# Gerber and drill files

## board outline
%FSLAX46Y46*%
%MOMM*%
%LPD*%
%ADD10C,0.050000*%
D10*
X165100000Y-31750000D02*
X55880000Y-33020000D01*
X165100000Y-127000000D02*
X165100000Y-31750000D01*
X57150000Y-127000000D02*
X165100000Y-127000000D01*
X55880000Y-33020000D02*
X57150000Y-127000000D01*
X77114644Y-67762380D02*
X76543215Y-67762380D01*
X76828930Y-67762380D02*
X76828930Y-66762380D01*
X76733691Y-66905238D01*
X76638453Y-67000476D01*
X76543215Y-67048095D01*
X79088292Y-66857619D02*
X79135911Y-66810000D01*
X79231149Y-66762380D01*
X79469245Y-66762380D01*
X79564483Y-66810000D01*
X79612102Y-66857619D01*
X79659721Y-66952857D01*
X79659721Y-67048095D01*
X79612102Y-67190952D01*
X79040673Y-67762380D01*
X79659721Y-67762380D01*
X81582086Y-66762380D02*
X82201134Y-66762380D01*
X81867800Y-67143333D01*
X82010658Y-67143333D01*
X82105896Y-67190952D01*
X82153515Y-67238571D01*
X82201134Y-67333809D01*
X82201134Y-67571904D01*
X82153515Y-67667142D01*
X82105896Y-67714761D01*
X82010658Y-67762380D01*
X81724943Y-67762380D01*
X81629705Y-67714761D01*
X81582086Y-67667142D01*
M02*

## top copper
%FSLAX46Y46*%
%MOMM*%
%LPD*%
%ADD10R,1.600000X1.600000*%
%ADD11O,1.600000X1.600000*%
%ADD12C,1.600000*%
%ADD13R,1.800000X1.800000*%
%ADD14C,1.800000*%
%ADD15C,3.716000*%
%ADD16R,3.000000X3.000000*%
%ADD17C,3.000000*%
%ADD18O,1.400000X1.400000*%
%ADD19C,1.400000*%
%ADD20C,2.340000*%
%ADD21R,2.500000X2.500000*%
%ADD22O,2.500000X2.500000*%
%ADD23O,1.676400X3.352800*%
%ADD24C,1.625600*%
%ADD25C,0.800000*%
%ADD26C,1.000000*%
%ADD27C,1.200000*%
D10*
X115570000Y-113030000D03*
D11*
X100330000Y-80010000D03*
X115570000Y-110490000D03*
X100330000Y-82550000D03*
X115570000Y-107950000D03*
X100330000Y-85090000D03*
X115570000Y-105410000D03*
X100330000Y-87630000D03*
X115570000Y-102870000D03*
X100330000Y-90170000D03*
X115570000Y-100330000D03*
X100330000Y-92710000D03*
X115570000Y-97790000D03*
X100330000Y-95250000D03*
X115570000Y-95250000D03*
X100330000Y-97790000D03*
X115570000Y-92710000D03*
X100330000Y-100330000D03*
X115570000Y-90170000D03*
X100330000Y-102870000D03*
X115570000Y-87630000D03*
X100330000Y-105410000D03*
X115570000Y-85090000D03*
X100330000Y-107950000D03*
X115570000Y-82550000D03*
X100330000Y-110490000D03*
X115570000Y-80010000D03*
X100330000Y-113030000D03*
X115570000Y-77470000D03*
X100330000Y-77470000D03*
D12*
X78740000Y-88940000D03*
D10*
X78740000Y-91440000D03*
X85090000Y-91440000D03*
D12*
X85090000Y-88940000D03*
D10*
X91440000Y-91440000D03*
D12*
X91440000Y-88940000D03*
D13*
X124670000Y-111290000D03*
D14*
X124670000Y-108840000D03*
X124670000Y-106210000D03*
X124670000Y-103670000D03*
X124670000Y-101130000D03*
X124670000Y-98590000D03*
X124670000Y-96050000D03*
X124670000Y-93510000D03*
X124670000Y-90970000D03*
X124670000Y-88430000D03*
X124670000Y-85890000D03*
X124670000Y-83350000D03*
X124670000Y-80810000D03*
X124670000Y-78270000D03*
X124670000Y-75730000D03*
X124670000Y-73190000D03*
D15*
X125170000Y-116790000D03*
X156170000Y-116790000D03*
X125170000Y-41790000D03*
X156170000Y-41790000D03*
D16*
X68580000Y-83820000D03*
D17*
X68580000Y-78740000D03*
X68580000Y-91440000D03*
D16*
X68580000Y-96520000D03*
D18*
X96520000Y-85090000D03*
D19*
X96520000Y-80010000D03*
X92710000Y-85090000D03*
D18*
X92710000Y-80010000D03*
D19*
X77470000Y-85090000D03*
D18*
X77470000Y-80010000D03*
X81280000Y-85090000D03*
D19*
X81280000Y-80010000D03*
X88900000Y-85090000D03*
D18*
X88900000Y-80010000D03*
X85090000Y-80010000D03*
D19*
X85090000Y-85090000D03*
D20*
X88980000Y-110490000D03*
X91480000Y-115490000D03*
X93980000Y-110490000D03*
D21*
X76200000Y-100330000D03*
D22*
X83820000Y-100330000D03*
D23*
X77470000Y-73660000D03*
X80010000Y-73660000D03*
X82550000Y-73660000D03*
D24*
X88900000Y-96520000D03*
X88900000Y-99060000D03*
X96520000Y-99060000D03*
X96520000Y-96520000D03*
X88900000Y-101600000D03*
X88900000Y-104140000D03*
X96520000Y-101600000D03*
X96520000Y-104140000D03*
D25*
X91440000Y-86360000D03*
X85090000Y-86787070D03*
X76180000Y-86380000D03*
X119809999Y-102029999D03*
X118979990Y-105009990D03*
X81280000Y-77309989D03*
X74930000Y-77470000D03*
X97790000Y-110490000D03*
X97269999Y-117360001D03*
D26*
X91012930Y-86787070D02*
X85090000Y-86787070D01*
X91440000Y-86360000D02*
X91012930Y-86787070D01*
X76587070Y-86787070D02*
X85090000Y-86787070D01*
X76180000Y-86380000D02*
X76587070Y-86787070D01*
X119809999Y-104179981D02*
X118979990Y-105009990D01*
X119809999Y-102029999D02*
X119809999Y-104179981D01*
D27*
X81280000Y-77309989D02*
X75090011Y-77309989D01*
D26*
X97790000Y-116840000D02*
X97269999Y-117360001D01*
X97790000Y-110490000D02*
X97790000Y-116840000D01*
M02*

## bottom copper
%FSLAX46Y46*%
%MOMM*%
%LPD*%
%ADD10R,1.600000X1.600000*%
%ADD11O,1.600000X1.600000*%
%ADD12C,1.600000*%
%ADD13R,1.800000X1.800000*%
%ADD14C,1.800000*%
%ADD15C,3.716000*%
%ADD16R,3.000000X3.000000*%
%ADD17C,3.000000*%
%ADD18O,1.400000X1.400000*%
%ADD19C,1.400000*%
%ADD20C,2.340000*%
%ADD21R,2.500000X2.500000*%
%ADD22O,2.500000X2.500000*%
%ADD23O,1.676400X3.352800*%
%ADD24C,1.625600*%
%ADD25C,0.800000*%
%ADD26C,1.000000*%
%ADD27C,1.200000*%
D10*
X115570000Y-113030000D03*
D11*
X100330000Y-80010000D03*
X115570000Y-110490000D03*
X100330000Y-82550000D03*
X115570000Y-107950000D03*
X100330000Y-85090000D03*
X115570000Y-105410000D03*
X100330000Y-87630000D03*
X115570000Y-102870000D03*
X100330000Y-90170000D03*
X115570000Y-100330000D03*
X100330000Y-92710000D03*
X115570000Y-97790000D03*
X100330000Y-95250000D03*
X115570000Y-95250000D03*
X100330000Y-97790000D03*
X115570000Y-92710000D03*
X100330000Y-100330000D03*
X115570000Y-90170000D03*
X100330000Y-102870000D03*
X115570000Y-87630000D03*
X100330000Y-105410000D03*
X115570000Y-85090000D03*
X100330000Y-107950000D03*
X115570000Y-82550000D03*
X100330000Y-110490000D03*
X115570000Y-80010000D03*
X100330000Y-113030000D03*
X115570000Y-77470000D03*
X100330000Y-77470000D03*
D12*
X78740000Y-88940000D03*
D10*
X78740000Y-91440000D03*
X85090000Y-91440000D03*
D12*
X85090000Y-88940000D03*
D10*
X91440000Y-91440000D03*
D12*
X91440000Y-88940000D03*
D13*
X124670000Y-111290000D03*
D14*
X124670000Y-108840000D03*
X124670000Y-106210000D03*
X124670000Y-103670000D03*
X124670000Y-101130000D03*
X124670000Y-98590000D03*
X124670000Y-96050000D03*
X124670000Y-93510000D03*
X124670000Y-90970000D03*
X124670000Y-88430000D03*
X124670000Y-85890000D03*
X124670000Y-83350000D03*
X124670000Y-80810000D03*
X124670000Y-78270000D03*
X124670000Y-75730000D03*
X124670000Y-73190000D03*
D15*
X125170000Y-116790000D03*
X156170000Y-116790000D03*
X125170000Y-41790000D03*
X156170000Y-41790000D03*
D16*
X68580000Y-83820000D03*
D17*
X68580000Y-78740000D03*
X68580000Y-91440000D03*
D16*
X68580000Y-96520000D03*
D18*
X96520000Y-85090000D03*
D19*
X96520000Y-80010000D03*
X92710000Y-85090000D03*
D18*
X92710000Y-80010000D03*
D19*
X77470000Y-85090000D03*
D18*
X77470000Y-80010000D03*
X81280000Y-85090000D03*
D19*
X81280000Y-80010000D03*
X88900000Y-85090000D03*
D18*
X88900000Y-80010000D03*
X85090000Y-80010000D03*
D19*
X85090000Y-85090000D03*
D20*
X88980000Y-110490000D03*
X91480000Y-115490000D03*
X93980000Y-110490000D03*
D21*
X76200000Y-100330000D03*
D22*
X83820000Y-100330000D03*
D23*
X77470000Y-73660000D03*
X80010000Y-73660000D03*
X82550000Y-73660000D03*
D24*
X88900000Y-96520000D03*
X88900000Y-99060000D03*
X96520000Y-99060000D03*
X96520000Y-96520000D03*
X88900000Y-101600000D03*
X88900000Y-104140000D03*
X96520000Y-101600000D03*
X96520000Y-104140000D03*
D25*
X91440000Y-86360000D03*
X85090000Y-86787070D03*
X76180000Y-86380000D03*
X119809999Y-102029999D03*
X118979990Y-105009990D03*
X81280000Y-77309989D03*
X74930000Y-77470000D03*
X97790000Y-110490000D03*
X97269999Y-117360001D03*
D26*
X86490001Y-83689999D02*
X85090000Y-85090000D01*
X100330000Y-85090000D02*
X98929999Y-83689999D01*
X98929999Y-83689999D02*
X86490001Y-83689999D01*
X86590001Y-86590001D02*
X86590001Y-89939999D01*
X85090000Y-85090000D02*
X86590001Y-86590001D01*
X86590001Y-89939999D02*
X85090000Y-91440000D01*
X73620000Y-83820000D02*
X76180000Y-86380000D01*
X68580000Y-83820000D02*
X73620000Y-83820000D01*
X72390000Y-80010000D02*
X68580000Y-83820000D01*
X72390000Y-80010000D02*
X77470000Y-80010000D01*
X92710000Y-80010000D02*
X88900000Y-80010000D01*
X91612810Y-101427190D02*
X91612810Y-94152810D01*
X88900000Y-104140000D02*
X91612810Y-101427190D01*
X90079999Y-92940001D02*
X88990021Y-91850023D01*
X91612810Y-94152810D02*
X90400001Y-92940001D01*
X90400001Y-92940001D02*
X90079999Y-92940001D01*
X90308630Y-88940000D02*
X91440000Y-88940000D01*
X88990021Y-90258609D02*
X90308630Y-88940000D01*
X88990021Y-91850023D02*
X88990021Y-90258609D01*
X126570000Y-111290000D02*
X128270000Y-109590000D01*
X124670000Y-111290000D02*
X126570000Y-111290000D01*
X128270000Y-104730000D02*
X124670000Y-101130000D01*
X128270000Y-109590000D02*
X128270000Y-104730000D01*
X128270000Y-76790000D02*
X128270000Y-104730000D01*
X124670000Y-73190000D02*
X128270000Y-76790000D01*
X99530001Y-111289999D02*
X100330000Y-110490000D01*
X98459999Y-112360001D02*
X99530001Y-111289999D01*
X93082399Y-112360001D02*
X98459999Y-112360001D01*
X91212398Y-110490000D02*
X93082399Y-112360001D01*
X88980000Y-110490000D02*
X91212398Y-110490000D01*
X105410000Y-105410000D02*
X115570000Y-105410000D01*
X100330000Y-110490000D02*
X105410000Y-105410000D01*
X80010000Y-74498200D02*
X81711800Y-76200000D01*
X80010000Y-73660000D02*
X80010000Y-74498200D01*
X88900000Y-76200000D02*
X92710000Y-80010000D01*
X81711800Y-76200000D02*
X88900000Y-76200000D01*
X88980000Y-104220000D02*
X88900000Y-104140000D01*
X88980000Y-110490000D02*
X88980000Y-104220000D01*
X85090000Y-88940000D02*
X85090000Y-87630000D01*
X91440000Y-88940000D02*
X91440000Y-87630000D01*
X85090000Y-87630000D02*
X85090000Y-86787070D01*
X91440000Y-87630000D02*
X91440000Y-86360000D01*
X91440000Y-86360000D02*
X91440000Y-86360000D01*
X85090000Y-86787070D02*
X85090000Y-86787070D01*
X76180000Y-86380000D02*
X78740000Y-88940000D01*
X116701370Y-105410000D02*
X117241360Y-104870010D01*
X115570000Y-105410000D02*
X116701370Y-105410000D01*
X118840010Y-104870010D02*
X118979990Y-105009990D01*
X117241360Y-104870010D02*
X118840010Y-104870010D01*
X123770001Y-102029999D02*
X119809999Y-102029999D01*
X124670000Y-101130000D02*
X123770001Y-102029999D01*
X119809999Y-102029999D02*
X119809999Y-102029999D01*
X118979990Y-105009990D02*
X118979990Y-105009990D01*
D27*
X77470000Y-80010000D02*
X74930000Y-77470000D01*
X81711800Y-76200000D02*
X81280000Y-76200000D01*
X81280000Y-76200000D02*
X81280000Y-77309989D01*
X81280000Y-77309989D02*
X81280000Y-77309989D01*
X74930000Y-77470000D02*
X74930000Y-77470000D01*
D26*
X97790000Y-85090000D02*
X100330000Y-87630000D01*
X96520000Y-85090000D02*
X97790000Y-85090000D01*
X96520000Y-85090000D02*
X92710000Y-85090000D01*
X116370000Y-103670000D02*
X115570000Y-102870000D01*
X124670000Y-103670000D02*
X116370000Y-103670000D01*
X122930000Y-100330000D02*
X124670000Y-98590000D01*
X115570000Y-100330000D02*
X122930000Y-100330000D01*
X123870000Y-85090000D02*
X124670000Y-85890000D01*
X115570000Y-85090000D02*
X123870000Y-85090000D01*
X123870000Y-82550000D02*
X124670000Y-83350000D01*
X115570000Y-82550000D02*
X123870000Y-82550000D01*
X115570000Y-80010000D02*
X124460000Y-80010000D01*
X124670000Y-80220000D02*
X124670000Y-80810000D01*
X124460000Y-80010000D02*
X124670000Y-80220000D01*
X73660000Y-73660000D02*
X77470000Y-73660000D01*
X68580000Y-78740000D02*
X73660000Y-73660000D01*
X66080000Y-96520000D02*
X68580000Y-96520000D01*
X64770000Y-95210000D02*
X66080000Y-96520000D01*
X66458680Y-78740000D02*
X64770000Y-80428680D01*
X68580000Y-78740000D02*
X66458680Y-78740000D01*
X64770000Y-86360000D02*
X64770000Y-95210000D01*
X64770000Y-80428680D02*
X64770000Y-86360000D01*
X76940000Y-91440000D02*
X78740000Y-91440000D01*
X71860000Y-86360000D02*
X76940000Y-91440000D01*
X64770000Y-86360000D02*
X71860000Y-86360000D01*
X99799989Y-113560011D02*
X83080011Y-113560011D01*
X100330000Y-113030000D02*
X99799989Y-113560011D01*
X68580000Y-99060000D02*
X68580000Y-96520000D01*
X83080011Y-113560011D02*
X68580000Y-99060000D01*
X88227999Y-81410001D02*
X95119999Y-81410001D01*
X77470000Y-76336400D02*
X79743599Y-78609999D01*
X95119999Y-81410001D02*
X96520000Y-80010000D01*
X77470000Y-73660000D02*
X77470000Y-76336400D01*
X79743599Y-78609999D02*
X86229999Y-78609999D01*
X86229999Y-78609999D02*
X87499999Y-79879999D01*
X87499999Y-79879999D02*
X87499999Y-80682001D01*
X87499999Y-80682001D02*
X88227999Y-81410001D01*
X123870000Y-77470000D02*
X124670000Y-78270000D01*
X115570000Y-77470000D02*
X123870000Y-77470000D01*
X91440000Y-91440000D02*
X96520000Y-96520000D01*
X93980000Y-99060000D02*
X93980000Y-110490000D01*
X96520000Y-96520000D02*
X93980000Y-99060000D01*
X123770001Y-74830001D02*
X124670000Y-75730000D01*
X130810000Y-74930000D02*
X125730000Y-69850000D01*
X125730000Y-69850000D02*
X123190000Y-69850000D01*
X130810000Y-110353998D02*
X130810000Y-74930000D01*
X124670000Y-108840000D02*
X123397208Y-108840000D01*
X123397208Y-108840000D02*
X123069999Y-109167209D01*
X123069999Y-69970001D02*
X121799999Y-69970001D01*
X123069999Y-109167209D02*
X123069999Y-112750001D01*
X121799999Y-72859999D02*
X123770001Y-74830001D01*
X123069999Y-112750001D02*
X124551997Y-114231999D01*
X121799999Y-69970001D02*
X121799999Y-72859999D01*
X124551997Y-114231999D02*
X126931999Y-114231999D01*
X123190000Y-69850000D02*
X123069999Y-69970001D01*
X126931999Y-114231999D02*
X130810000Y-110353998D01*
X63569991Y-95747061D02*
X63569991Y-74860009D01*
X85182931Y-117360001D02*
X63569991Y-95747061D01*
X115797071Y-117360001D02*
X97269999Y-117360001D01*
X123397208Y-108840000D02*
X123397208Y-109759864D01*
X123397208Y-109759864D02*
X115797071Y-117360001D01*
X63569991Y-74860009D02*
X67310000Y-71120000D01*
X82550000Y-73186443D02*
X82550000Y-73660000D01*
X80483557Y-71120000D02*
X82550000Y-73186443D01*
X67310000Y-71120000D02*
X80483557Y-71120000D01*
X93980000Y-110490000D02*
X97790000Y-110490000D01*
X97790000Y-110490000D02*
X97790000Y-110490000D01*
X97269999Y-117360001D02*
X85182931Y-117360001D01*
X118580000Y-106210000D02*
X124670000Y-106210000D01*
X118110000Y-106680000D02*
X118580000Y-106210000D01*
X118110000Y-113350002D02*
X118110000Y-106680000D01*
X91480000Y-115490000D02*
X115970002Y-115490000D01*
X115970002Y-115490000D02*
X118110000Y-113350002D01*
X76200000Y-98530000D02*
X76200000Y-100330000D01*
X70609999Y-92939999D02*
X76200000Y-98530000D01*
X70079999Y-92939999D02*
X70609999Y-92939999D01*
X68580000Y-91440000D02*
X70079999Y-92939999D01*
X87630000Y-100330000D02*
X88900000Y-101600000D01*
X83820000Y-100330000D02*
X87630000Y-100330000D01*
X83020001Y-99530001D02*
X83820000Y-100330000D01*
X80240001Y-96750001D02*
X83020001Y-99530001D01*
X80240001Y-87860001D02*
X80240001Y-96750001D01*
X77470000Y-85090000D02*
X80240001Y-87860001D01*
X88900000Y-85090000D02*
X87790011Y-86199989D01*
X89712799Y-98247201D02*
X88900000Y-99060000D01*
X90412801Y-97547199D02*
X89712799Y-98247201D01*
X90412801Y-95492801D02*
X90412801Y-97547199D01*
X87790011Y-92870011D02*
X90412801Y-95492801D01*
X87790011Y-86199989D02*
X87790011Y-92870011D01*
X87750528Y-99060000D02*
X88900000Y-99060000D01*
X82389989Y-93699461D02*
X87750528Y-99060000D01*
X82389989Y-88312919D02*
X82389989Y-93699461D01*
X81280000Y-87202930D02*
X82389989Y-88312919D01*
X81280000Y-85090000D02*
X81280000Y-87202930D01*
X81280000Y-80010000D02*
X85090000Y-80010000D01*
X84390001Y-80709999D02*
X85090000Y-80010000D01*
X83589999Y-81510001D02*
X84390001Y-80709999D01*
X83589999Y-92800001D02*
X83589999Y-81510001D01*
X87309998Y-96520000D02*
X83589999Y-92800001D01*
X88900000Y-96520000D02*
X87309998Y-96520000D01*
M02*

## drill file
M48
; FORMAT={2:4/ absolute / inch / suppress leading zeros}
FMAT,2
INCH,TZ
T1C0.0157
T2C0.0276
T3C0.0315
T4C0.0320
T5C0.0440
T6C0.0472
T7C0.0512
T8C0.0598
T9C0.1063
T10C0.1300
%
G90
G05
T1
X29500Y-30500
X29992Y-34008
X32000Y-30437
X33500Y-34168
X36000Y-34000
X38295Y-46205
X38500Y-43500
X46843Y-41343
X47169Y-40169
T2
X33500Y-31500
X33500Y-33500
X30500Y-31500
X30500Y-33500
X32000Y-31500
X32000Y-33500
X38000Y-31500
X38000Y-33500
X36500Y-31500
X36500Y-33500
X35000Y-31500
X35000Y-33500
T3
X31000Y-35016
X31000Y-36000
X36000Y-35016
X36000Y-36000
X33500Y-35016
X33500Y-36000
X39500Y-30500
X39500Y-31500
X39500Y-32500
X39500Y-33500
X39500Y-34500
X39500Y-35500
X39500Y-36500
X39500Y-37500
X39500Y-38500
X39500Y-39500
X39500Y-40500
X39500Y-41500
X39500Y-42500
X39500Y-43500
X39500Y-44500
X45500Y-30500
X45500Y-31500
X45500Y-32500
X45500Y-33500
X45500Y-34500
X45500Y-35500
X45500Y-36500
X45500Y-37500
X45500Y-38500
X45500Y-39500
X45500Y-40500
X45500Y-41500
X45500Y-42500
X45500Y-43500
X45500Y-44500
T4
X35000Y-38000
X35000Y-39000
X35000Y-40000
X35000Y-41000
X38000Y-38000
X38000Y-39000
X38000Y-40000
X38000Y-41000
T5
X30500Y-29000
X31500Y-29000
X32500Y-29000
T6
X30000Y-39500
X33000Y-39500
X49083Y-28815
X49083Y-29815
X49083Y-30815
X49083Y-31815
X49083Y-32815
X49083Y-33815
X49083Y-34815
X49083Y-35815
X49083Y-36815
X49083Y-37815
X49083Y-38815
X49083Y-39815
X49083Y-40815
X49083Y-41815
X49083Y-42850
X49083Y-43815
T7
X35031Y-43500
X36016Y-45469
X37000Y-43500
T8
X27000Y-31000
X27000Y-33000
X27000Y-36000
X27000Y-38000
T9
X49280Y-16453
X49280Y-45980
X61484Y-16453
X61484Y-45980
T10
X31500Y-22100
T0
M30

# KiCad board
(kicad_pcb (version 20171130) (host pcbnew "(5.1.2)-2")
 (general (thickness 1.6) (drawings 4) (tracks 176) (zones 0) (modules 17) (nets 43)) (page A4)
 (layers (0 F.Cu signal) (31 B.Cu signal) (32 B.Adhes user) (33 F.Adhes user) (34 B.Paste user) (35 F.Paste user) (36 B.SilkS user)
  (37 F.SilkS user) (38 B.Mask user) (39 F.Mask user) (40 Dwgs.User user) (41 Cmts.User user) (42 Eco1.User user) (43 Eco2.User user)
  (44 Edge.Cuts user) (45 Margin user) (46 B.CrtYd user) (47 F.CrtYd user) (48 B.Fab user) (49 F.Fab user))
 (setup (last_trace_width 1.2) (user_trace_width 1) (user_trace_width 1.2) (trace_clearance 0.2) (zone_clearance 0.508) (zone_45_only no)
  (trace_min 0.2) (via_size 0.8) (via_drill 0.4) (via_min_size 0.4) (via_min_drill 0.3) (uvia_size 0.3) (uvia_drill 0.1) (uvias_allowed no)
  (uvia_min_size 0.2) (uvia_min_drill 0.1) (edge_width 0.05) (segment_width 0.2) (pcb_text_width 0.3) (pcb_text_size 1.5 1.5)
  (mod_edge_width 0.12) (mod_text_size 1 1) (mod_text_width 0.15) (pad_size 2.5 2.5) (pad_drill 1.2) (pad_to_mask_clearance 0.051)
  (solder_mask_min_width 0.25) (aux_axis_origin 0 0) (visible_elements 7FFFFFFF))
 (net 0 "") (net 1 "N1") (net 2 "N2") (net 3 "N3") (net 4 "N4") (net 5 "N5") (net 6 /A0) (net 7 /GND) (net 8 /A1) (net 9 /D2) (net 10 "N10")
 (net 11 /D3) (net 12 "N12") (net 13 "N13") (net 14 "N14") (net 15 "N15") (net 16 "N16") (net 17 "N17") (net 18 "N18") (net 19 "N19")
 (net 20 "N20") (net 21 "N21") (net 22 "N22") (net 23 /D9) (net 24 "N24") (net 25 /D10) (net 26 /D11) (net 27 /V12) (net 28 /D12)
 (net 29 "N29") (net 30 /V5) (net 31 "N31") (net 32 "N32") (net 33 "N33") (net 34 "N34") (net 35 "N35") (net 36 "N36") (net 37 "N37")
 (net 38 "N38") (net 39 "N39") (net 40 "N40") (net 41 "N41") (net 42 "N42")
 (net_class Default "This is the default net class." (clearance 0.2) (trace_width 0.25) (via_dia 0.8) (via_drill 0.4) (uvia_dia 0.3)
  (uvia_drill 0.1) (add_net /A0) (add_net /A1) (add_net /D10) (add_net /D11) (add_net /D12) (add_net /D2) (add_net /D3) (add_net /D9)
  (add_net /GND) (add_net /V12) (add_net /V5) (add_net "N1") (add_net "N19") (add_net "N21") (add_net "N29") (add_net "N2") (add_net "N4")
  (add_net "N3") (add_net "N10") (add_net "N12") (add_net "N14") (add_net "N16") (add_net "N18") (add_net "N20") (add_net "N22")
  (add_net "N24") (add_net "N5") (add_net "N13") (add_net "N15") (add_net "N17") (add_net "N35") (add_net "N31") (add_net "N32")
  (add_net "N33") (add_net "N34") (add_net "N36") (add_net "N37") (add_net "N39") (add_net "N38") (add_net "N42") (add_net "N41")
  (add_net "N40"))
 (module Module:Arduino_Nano (layer F.Cu) (at 115.57 113.03 180)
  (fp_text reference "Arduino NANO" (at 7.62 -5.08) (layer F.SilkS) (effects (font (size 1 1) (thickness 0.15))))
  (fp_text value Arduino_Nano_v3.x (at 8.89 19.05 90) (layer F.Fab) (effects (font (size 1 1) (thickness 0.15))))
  (pad 1 thru_hole rect (at 0 0 180) (size 1.6 1.6) (drill 0.8) (layers *.Cu *.Mask) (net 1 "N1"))
  (pad 17 thru_hole oval (at 15.24 33.02 180) (size 1.6 1.6) (drill 0.8) (layers *.Cu *.Mask) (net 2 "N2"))
  (pad 2 thru_hole oval (at 0 2.54 180) (size 1.6 1.6) (drill 0.8) (layers *.Cu *.Mask) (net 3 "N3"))
  (pad 18 thru_hole oval (at 15.24 30.48 180) (size 1.6 1.6) (drill 0.8) (layers *.Cu *.Mask) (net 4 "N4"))
  (pad 3 thru_hole oval (at 0 5.08 180) (size 1.6 1.6) (drill 0.8) (layers *.Cu *.Mask) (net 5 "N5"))
  (pad 19 thru_hole oval (at 15.24 27.94 180) (size 1.6 1.6) (drill 0.8) (layers *.Cu *.Mask) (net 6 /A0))
  (pad 4 thru_hole oval (at 0 7.62 180) (size 1.6 1.6) (drill 0.8) (layers *.Cu *.Mask) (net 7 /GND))
  (pad 20 thru_hole oval (at 15.24 25.4 180) (size 1.6 1.6) (drill 0.8) (layers *.Cu *.Mask) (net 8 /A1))
  (pad 5 thru_hole oval (at 0 10.16 180) (size 1.6 1.6) (drill 0.8) (layers *.Cu *.Mask) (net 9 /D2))
  (pad 21 thru_hole oval (at 15.24 22.86 180) (size 1.6 1.6) (drill 0.8) (layers *.Cu *.Mask) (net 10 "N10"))
  (pad 6 thru_hole oval (at 0 12.7 180) (size 1.6 1.6) (drill 0.8) (layers *.Cu *.Mask) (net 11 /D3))
  (pad 22 thru_hole oval (at 15.24 20.32 180) (size 1.6 1.6) (drill 0.8) (layers *.Cu *.Mask) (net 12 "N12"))
  (pad 7 thru_hole oval (at 0 15.24 180) (size 1.6 1.6) (drill 0.8) (layers *.Cu *.Mask) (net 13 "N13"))
  (pad 23 thru_hole oval (at 15.24 17.78 180) (size 1.6 1.6) (drill 0.8) (layers *.Cu *.Mask) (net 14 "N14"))
  (pad 8 thru_hole oval (at 0 17.78 180) (size 1.6 1.6) (drill 0.8) (layers *.Cu *.Mask) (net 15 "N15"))
  (pad 24 thru_hole oval (at 15.24 15.24 180) (size 1.6 1.6) (drill 0.8) (layers *.Cu *.Mask) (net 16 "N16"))
  (pad 9 thru_hole oval (at 0 20.32 180) (size 1.6 1.6) (drill 0.8) (layers *.Cu *.Mask) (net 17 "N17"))
  (pad 25 thru_hole oval (at 15.24 12.7 180) (size 1.6 1.6) (drill 0.8) (layers *.Cu *.Mask) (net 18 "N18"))
  (pad 10 thru_hole oval (at 0 22.86 180) (size 1.6 1.6) (drill 0.8) (layers *.Cu *.Mask) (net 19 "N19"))
  (pad 26 thru_hole oval (at 15.24 10.16 180) (size 1.6 1.6) (drill 0.8) (layers *.Cu *.Mask) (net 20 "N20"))
  (pad 11 thru_hole oval (at 0 25.4 180) (size 1.6 1.6) (drill 0.8) (layers *.Cu *.Mask) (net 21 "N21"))
  (pad 27 thru_hole oval (at 15.24 7.62 180) (size 1.6 1.6) (drill 0.8) (layers *.Cu *.Mask) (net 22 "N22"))
  (pad 12 thru_hole oval (at 0 27.94 180) (size 1.6 1.6) (drill 0.8) (layers *.Cu *.Mask) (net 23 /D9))
  (pad 28 thru_hole oval (at 15.24 5.08 180) (size 1.6 1.6) (drill 0.8) (layers *.Cu *.Mask) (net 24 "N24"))
  (pad 13 thru_hole oval (at 0 30.48 180) (size 1.6 1.6) (drill 0.8) (layers *.Cu *.Mask) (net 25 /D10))
  (pad 29 thru_hole oval (at 15.24 2.54 180) (size 1.6 1.6) (drill 0.8) (layers *.Cu *.Mask) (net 7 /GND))
  (pad 14 thru_hole oval (at 0 33.02 180) (size 1.6 1.6) (drill 0.8) (layers *.Cu *.Mask) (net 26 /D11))
  (pad 30 thru_hole oval (at 15.24 0 180) (size 1.6 1.6) (drill 0.8) (layers *.Cu *.Mask) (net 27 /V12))
  (pad 15 thru_hole oval (at 0 35.56 180) (size 1.6 1.6) (drill 0.8) (layers *.Cu *.Mask) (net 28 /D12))
  (pad 16 thru_hole oval (at 15.24 35.56 180) (size 1.6 1.6) (drill 0.8) (layers *.Cu *.Mask) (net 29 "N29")))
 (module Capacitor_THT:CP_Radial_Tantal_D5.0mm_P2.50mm (layer F.Cu) (at 78.74 91.44 90)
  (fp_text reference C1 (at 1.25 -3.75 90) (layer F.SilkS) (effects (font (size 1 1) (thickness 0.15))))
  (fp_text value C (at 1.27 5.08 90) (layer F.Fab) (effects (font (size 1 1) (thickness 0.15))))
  (pad 2 thru_hole circle (at 2.5 0 90) (size 1.6 1.6) (drill 0.8) (layers *.Cu *.Mask) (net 7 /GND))
  (pad 1 thru_hole rect (at 0 0 90) (size 1.6 1.6) (drill 0.8) (layers *.Cu *.Mask) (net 27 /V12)))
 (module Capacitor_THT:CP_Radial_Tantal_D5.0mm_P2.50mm (layer F.Cu) (at 85.09 91.44 90)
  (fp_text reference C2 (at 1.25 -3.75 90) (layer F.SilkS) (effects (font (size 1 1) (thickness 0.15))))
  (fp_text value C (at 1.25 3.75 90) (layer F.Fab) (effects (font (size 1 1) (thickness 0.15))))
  (pad 1 thru_hole rect (at 0 0 90) (size 1.6 1.6) (drill 0.8) (layers *.Cu *.Mask) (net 6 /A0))
  (pad 2 thru_hole circle (at 2.5 0 90) (size 1.6 1.6) (drill 0.8) (layers *.Cu *.Mask) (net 7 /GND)))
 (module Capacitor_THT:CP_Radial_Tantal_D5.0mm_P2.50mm (layer F.Cu) (at 91.44 91.44 90)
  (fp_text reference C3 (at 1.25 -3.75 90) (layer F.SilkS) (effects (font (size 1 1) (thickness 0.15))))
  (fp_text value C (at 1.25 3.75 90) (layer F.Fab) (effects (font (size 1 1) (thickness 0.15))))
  (pad 1 thru_hole rect (at 0 0 90) (size 1.6 1.6) (drill 0.8) (layers *.Cu *.Mask) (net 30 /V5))
  (pad 2 thru_hole circle (at 2.5 0 90) (size 1.6 1.6) (drill 0.8) (layers *.Cu *.Mask) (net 7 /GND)))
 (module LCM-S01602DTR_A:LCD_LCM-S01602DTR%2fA (layer F.Cu) (at 140.97 78.74 90)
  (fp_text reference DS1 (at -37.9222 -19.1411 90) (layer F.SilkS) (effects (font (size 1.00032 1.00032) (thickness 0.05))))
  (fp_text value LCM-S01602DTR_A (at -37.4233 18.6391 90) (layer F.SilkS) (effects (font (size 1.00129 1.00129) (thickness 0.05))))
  (pad 1 thru_hole rect (at -32.55 -16.3 90) (size 1.8 1.8) (drill 1.2) (layers *.Cu *.Mask) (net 7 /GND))
  (pad 2 thru_hole circle (at -30.1 -16.3 90) (size 1.8 1.8) (drill 1.2) (layers *.Cu *.Mask) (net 30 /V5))
  (pad 3 thru_hole circle (at -27.47 -16.3 90) (size 1.8 1.8) (drill 1.2) (layers *.Cu *.Mask) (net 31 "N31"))
  (pad 4 thru_hole circle (at -24.93 -16.3 90) (size 1.8 1.8) (drill 1.2) (layers *.Cu *.Mask) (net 9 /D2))
  (pad 5 thru_hole circle (at -22.39 -16.3 90) (size 1.8 1.8) (drill 1.2) (layers *.Cu *.Mask) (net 7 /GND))
  (pad 6 thru_hole circle (at -19.85 -16.3 90) (size 1.8 1.8) (drill 1.2) (layers *.Cu *.Mask) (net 11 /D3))
  (pad 7 thru_hole circle (at -17.31 -16.3 90) (size 1.8 1.8) (drill 1.2) (layers *.Cu *.Mask) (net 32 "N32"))
  (pad 8 thru_hole circle (at -14.77 -16.3 90) (size 1.8 1.8) (drill 1.2) (layers *.Cu *.Mask) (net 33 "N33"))
  (pad 9 thru_hole circle (at -12.23 -16.3 90) (size 1.8 1.8) (drill 1.2) (layers *.Cu *.Mask) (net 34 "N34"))
  (pad 10 thru_hole circle (at -9.69 -16.3 90) (size 1.8 1.8) (drill 1.2) (layers *.Cu *.Mask) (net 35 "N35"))
  (pad 11 thru_hole circle (at -7.15 -16.3 90) (size 1.8 1.8) (drill 1.2) (layers *.Cu *.Mask) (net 23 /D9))
  (pad 12 thru_hole circle (at -4.61 -16.3 90) (size 1.8 1.8) (drill 1.2) (layers *.Cu *.Mask) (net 25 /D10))
  (pad 13 thru_hole circle (at -2.07 -16.3 90) (size 1.8 1.8) (drill 1.2) (layers *.Cu *.Mask) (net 26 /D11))
  (pad 14 thru_hole circle (at 0.47 -16.3 90) (size 1.8 1.8) (drill 1.2) (layers *.Cu *.Mask) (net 28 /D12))
  (pad 15 thru_hole circle (at 3.01 -16.3 90) (size 1.8 1.8) (drill 1.2) (layers *.Cu *.Mask) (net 30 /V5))
  (pad 16 thru_hole circle (at 5.55 -16.3 90) (size 1.8 1.8) (drill 1.2) (layers *.Cu *.Mask) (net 7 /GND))
  (pad 17 thru_hole circle (at -38.05 -15.8 90) (size 3.716 3.716) (drill 2.7) (layers *.Cu *.Mask))
  (pad 18 thru_hole circle (at -38.05 15.2 90) (size 3.716 3.716) (drill 2.7) (layers *.Cu *.Mask))
  (pad 19 thru_hole circle (at 36.95 -15.8 90) (size 3.716 3.716) (drill 2.7) (layers *.Cu *.Mask))
  (pad 20 thru_hole circle (at 36.95 15.2 90) (size 3.716 3.716) (drill 2.7) (layers *.Cu *.Mask)))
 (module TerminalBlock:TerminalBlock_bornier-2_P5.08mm (layer F.Cu) (at 68.58 83.82 90)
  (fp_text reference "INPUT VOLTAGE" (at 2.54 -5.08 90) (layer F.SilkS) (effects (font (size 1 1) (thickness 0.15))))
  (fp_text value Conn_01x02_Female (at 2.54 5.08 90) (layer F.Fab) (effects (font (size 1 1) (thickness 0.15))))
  (pad 1 thru_hole rect (at 0 0 90) (size 3 3) (drill 1.52) (layers *.Cu *.Mask) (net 7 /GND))
  (pad 2 thru_hole circle (at 5.08 0 90) (size 3 3) (drill 1.52) (layers *.Cu *.Mask) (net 27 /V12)))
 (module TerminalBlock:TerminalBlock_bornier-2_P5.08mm (layer F.Cu) (at 68.58 96.52 90)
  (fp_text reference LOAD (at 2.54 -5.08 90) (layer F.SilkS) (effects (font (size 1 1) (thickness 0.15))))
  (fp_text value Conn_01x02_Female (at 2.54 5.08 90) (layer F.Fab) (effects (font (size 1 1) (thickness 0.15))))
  (pad 2 thru_hole circle (at 5.08 0 90) (size 3 3) (drill 1.52) (layers *.Cu *.Mask) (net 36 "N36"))
  (pad 1 thru_hole rect (at 0 0 90) (size 3 3) (drill 1.52) (layers *.Cu *.Mask) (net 27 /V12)))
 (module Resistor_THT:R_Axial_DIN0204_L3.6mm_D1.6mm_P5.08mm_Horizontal (layer F.Cu) (at 96.52 80.01 270)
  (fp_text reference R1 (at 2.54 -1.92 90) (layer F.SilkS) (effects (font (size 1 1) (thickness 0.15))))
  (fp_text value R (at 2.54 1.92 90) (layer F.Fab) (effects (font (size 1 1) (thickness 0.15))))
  (pad 2 thru_hole oval (at 5.08 0 270) (size 1.4 1.4) (drill 0.7) (layers *.Cu *.Mask) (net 8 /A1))
  (pad 1 thru_hole circle (at 0 0 270) (size 1.4 1.4) (drill 0.7) (layers *.Cu *.Mask) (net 27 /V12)))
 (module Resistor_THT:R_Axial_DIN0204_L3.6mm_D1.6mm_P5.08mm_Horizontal (layer F.Cu) (at 92.71 85.09 90)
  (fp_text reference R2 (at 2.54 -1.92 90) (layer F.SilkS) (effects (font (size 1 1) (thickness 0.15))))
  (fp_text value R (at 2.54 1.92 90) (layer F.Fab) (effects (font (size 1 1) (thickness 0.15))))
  (pad 1 thru_hole circle (at 0 0 90) (size 1.4 1.4) (drill 0.7) (layers *.Cu *.Mask) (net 8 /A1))
  (pad 2 thru_hole oval (at 5.08 0 90) (size 1.4 1.4) (drill 0.7) (layers *.Cu *.Mask) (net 7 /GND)))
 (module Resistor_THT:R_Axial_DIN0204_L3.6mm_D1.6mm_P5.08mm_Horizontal (layer F.Cu) (at 77.47 85.09 90)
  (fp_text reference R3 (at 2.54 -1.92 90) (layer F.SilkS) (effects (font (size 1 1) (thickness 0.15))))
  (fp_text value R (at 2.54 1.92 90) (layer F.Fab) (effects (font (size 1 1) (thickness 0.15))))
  (pad 1 thru_hole circle (at 0 0 90) (size 1.4 1.4) (drill 0.7) (layers *.Cu *.Mask) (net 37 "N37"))
  (pad 2 thru_hole oval (at 5.08 0 90) (size 1.4 1.4) (drill 0.7) (layers *.Cu *.Mask) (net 7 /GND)))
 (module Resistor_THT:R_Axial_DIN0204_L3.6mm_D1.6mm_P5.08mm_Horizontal (layer F.Cu) (at 81.28 80.01 270)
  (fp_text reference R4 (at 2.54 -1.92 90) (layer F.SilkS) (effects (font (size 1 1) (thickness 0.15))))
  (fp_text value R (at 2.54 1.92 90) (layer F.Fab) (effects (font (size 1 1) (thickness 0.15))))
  (pad 2 thru_hole oval (at 5.08 0 270) (size 1.4 1.4) (drill 0.7) (layers *.Cu *.Mask) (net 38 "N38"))
  (pad 1 thru_hole circle (at 0 0 270) (size 1.4 1.4) (drill 0.7) (layers *.Cu *.Mask) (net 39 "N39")))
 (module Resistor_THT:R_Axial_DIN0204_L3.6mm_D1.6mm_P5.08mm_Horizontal (layer F.Cu) (at 88.9 85.09 90)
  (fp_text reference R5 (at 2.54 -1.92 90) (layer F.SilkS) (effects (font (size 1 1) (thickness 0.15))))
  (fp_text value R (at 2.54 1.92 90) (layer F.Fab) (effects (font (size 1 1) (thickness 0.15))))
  (pad 1 thru_hole circle (at 0 0 90) (size 1.4 1.4) (drill 0.7) (layers *.Cu *.Mask) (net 38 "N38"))
  (pad 2 thru_hole oval (at 5.08 0 90) (size 1.4 1.4) (drill 0.7) (layers *.Cu *.Mask) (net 7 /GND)))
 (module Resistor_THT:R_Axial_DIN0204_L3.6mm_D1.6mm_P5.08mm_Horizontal (layer F.Cu) (at 85.09 85.09 90)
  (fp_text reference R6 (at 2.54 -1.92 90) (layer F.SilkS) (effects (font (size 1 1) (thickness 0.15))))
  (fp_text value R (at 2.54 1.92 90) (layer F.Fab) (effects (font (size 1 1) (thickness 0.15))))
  (pad 2 thru_hole oval (at 5.08 0 90) (size 1.4 1.4) (drill 0.7) (layers *.Cu *.Mask) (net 39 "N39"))
  (pad 1 thru_hole circle (at 0 0 90) (size 1.4 1.4) (drill 0.7) (layers *.Cu *.Mask) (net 6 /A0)))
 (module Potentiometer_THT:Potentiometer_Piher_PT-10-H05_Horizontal (layer F.Cu) (at 93.98 110.49 270)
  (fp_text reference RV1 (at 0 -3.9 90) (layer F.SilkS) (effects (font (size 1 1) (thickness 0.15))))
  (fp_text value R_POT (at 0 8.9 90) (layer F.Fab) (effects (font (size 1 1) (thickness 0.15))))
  (pad 3 thru_hole circle (at 0 5 270) (size 2.34 2.34) (drill 1.3) (layers *.Cu *.Mask) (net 7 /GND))
  (pad 2 thru_hole circle (at 5 2.5 270) (size 2.34 2.34) (drill 1.3) (layers *.Cu *.Mask) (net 31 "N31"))
  (pad 1 thru_hole circle (at 0 0 270) (size 2.34 2.34) (drill 1.3) (layers *.Cu *.Mask) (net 30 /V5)))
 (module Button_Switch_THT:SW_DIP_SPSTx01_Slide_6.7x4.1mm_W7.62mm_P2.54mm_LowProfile (layer F.Cu) (at 76.2 100.33)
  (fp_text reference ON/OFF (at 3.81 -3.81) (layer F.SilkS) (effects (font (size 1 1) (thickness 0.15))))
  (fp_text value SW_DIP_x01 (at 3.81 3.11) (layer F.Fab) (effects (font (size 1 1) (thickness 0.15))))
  (pad 1 thru_hole rect (at 0 0) (size 2.5 2.5) (drill 1.2) (layers *.Cu *.Mask) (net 36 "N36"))
  (pad 2 thru_hole oval (at 7.62 0) (size 2.5 2.5) (drill 1.2) (layers *.Cu *.Mask) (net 37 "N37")))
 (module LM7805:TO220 (layer F.Cu) (at 80.01 67.31)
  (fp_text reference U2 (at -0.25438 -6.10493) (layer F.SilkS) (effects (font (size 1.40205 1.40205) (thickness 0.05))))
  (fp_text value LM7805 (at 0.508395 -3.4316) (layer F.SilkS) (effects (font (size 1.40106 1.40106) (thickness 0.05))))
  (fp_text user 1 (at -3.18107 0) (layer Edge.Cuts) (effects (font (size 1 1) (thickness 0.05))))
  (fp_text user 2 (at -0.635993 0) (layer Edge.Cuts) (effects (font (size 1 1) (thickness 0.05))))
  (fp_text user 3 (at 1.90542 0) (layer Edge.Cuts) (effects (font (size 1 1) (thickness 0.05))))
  (pad 1 thru_hole oval (at -2.54 6.35 90) (size 3.3528 1.6764) (drill 1.1176) (layers *.Cu *.Mask) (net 27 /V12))
  (pad 2 thru_hole oval (at 0 6.35 90) (size 3.3528 1.6764) (drill 1.1176) (layers *.Cu *.Mask) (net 7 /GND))
  (pad 3 thru_hole oval (at 2.54 6.35 90) (size 3.3528 1.6764) (drill 1.1176) (layers *.Cu *.Mask) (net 30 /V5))
  (pad Hole np_thru_hole circle (at 0 -11.176) (size 3.302 3.302) (drill 3.302) (layers *.Cu *.Mask F.SilkS)))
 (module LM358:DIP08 (layer F.Cu) (at 92.71 100.33 270)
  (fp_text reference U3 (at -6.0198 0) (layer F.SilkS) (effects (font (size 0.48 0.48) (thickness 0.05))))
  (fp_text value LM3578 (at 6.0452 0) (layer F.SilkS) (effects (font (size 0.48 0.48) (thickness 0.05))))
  (pad 1 thru_hole circle (at -3.81 3.81) (size 1.6256 1.6256) (drill 0.8128) (layers *.Cu *.Mask) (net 39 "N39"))
  (pad 2 thru_hole circle (at -1.27 3.81) (size 1.6256 1.6256) (drill 0.8128) (layers *.Cu *.Mask) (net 38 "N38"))
  (pad 7 thru_hole circle (at -1.27 -3.81) (size 1.6256 1.6256) (drill 0.8128) (layers *.Cu *.Mask) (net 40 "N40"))
  (pad 8 thru_hole circle (at -3.81 -3.81) (size 1.6256 1.6256) (drill 0.8128) (layers *.Cu *.Mask) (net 30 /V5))
  (pad 3 thru_hole circle (at 1.27 3.81) (size 1.6256 1.6256) (drill 0.8128) (layers *.Cu *.Mask) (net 37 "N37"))
  (pad 4 thru_hole circle (at 3.81 3.81) (size 1.6256 1.6256) (drill 0.8128) (layers *.Cu *.Mask) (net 7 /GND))
  (pad 6 thru_hole circle (at 1.27 -3.81) (size 1.6256 1.6256) (drill 0.8128) (layers *.Cu *.Mask) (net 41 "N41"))
  (pad 5 thru_hole circle (at 3.81 -3.81) (size 1.6256 1.6256) (drill 0.8128) (layers *.Cu *.Mask) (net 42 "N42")))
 (gr_line (start 165.1 31.75) (end 55.88 33.02) (layer Edge.Cuts) (width 0.05))
 (gr_line (start 165.1 127) (end 165.1 31.75) (layer Edge.Cuts) (width 0.05))
 (gr_line (start 57.15 127) (end 165.1 127) (layer Edge.Cuts) (width 0.05))
 (gr_line (start 55.88 33.02) (end 57.15 127) (layer Edge.Cuts) (width 0.05))
 (segment (start 86.490001 83.689999) (end 85.09 85.09) (width 1) (layer B.Cu) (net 6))
 (segment (start 100.33 85.09) (end 98.929999 83.689999) (width 1) (layer B.Cu) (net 6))
 (segment (start 98.929999 83.689999) (end 86.490001 83.689999) (width 1) (layer B.Cu) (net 6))
 (segment (start 86.590001 86.590001) (end 86.590001 89.939999) (width 1) (layer B.Cu) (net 6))
 (segment (start 85.09 85.09) (end 86.590001 86.590001) (width 1) (layer B.Cu) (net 6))
 (segment (start 86.590001 89.939999) (end 85.09 91.44) (width 1) (layer B.Cu) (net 6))
 (segment (start 73.62 83.82) (end 76.18 86.38) (width 1) (layer B.Cu) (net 7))
 (segment (start 68.58 83.82) (end 73.62 83.82) (width 1) (layer B.Cu) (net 7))
 (segment (start 72.39 80.01) (end 68.58 83.82) (width 1) (layer B.Cu) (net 7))
 (segment (start 72.39 80.01) (end 77.47 80.01) (width 1) (layer B.Cu) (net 7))
 (segment (start 92.71 80.01) (end 88.9 80.01) (width 1) (layer B.Cu) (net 7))
 (segment (start 91.61281 101.42719) (end 91.61281 94.15281) (width 1) (layer B.Cu) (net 7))
 (segment (start 88.9 104.14) (end 91.61281 101.42719) (width 1) (layer B.Cu) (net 7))
 (segment (start 90.079999 92.940001) (end 88.990021 91.850023) (width 1) (layer B.Cu) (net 7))
 (segment (start 91.61281 94.15281) (end 90.400001 92.940001) (width 1) (layer B.Cu) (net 7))
 (segment (start 90.400001 92.940001) (end 90.079999 92.940001) (width 1) (layer B.Cu) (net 7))
 (segment (start 90.30863 88.94) (end 91.44 88.94) (width 1) (layer B.Cu) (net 7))
 (segment (start 88.990021 90.258609) (end 90.30863 88.94) (width 1) (layer B.Cu) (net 7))
 (segment (start 88.990021 91.850023) (end 88.990021 90.258609) (width 1) (layer B.Cu) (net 7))
 (segment (start 126.57 111.29) (end 128.27 109.59) (width 1) (layer B.Cu) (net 7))
 (segment (start 124.67 111.29) (end 126.57 111.29) (width 1) (layer B.Cu) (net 7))
 (segment (start 128.27 104.73) (end 124.67 101.13) (width 1) (layer B.Cu) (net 7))
 (segment (start 128.27 109.59) (end 128.27 104.73) (width 1) (layer B.Cu) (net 7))
 (segment (start 128.27 76.79) (end 128.27 104.73) (width 1) (layer B.Cu) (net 7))
 (segment (start 124.67 73.19) (end 128.27 76.79) (width 1) (layer B.Cu) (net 7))
 (segment (start 99.530001 111.289999) (end 100.33 110.49) (width 1) (layer B.Cu) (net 7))
 (segment (start 98.459999 112.360001) (end 99.530001 111.289999) (width 1) (layer B.Cu) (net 7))
 (segment (start 93.082399 112.360001) (end 98.459999 112.360001) (width 1) (layer B.Cu) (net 7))
 (segment (start 91.212398 110.49) (end 93.082399 112.360001) (width 1) (layer B.Cu) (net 7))
 (segment (start 88.98 110.49) (end 91.212398 110.49) (width 1) (layer B.Cu) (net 7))
 (segment (start 105.41 105.41) (end 115.57 105.41) (width 1) (layer B.Cu) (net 7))
 (segment (start 100.33 110.49) (end 105.41 105.41) (width 1) (layer B.Cu) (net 7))
 (segment (start 80.01 74.4982) (end 81.7118 76.2) (width 1) (layer B.Cu) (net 7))
 (segment (start 80.01 73.66) (end 80.01 74.4982) (width 1) (layer B.Cu) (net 7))
 (segment (start 88.9 76.2) (end 92.71 80.01) (width 1) (layer B.Cu) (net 7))
 (segment (start 81.7118 76.2) (end 88.9 76.2) (width 1) (layer B.Cu) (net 7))
 (segment (start 88.98 104.22) (end 88.9 104.14) (width 1) (layer B.Cu) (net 7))
 (segment (start 88.98 110.49) (end 88.98 104.22) (width 1) (layer B.Cu) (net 7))
 (segment (start 85.09 88.94) (end 85.09 87.63) (width 1) (layer B.Cu) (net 7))
 (segment (start 91.44 88.94) (end 91.44 87.63) (width 1) (layer B.Cu) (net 7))
 (segment (start 85.09 87.63) (end 85.09 86.78707) (width 1) (layer B.Cu) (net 7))
 (segment (start 91.44 87.63) (end 91.44 86.36) (width 1) (layer B.Cu) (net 7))
 (segment (start 91.44 86.36) (end 91.44 86.36) (width 1) (layer B.Cu) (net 7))
 (via (at 91.44 86.36) (size 0.8) (drill 0.4) (layers F.Cu B.Cu) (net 7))
 (segment (start 85.09 86.78707) (end 85.09 86.78707) (width 1) (layer B.Cu) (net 7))
 (via (at 85.09 86.78707) (size 0.8) (drill 0.4) (layers F.Cu B.Cu) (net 7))
 (segment (start 76.18 86.38) (end 78.74 88.94) (width 1) (layer B.Cu) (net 7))
 (via (at 76.18 86.38) (size 0.8) (drill 0.4) (layers F.Cu B.Cu) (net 7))
 (segment (start 91.01293 86.78707) (end 85.09 86.78707) (width 1) (layer F.Cu) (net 7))
 (segment (start 91.44 86.36) (end 91.01293 86.78707) (width 1) (layer F.Cu) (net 7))
 (segment (start 76.58707 86.78707) (end 85.09 86.78707) (width 1) (layer F.Cu) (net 7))
 (segment (start 76.18 86.38) (end 76.58707 86.78707) (width 1) (layer F.Cu) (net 7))
 (segment (start 116.70137 105.41) (end 117.24136 104.87001) (width 1) (layer B.Cu) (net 7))
 (segment (start 115.57 105.41) (end 116.70137 105.41) (width 1) (layer B.Cu) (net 7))
 (segment (start 118.84001 104.87001) (end 118.97999 105.00999) (width 1) (layer B.Cu) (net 7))
 (segment (start 117.24136 104.87001) (end 118.84001 104.87001) (width 1) (layer B.Cu) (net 7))
 (segment (start 123.770001 102.029999) (end 119.809999 102.029999) (width 1) (layer B.Cu) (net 7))
 (segment (start 124.67 101.13) (end 123.770001 102.029999) (width 1) (layer B.Cu) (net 7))
 (segment (start 119.809999 102.029999) (end 119.809999 102.029999) (width 1) (layer B.Cu) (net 7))
 (via (at 119.809999 102.029999) (size 0.8) (drill 0.4) (layers F.Cu B.Cu) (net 7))
 (segment (start 118.97999 105.00999) (end 118.97999 105.00999) (width 1) (layer B.Cu) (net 7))
 (via (at 118.97999 105.00999) (size 0.8) (drill 0.4) (layers F.Cu B.Cu) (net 7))
 (segment (start 119.809999 104.179981) (end 118.97999 105.00999) (width 1) (layer F.Cu) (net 7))
 (segment (start 119.809999 102.029999) (end 119.809999 104.179981) (width 1) (layer F.Cu) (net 7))
 (segment (start 77.47 80.01) (end 74.93 77.47) (width 1.2) (layer B.Cu) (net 7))
 (segment (start 81.7118 76.2) (end 81.28 76.2) (width 1.2) (layer B.Cu) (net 7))
 (segment (start 81.28 76.2) (end 81.28 77.309989) (width 1.2) (layer B.Cu) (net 7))
 (segment (start 81.28 77.309989) (end 81.28 77.309989) (width 1.2) (layer B.Cu) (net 7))
 (via (at 81.28 77.309989) (size 0.8) (drill 0.4) (layers F.Cu B.Cu) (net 7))
 (segment (start 74.93 77.47) (end 74.93 77.47) (width 1.2) (layer B.Cu) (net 7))
 (via (at 74.93 77.47) (size 0.8) (drill 0.4) (layers F.Cu B.Cu) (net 7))
 (segment (start 81.28 77.309989) (end 75.090011 77.309989) (width 1.2) (layer F.Cu) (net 7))
 (segment (start 97.79 85.09) (end 100.33 87.63) (width 1) (layer B.Cu) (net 8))
 (segment (start 96.52 85.09) (end 97.79 85.09) (width 1) (layer B.Cu) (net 8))
 (segment (start 96.52 85.09) (end 92.71 85.09) (width 1) (layer B.Cu) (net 8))
 (segment (start 116.37 103.67) (end 115.57 102.87) (width 1) (layer B.Cu) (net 9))
 (segment (start 124.67 103.67) (end 116.37 103.67) (width 1) (layer B.Cu) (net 9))
 (segment (start 122.93 100.33) (end 124.67 98.59) (width 1) (layer B.Cu) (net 11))
 (segment (start 115.57 100.33) (end 122.93 100.33) (width 1) (layer B.Cu) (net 11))
 (segment (start 123.87 85.09) (end 124.67 85.89) (width 1) (layer B.Cu) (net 23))
 (segment (start 115.57 85.09) (end 123.87 85.09) (width 1) (layer B.Cu) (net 23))
 (segment (start 123.87 82.55) (end 124.67 83.35) (width 1) (layer B.Cu) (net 25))
 (segment (start 115.57 82.55) (end 123.87 82.55) (width 1) (layer B.Cu) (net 25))
 (segment (start 115.57 80.01) (end 124.46 80.01) (width 1) (layer B.Cu) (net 26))
 (segment (start 124.67 80.22) (end 124.67 80.81) (width 1) (layer B.Cu) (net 26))
 (segment (start 124.46 80.01) (end 124.67 80.22) (width 1) (layer B.Cu) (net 26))
 (segment (start 73.66 73.66) (end 77.47 73.66) (width 1) (layer B.Cu) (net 27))
 (segment (start 68.58 78.74) (end 73.66 73.66) (width 1) (layer B.Cu) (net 27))
 (segment (start 66.08 96.52) (end 68.58 96.52) (width 1) (layer B.Cu) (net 27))
 (segment (start 64.77 95.21) (end 66.08 96.52) (width 1) (layer B.Cu) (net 27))
 (segment (start 66.45868 78.74) (end 64.77 80.42868) (width 1) (layer B.Cu) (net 27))
 (segment (start 68.58 78.74) (end 66.45868 78.74) (width 1) (layer B.Cu) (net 27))
 (segment (start 64.77 86.36) (end 64.77 95.21) (width 1) (layer B.Cu) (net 27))
 (segment (start 64.77 80.42868) (end 64.77 86.36) (width 1) (layer B.Cu) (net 27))
 (segment (start 76.94 91.44) (end 78.74 91.44) (width 1) (layer B.Cu) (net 27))
 (segment (start 71.86 86.36) (end 76.94 91.44) (width 1) (layer B.Cu) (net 27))
 (segment (start 64.77 86.36) (end 71.86 86.36) (width 1) (layer B.Cu) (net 27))
 (segment (start 99.799989 113.560011) (end 83.080011 113.560011) (width 1) (layer B.Cu) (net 27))
 (segment (start 100.33 113.03) (end 99.799989 113.560011) (width 1) (layer B.Cu) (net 27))
 (segment (start 68.58 99.06) (end 68.58 96.52) (width 1) (layer B.Cu) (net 27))
 (segment (start 83.080011 113.560011) (end 68.58 99.06) (width 1) (layer B.Cu) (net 27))
 (segment (start 88.227999 81.410001) (end 95.119999 81.410001) (width 1) (layer B.Cu) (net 27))
 (segment (start 77.47 76.3364) (end 79.743599 78.609999) (width 1) (layer B.Cu) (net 27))
 (segment (start 95.119999 81.410001) (end 96.52 80.01) (width 1) (layer B.Cu) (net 27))
 (segment (start 77.47 73.66) (end 77.47 76.3364) (width 1) (layer B.Cu) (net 27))
 (segment (start 79.743599 78.609999) (end 86.229999 78.609999) (width 1) (layer B.Cu) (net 27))
 (segment (start 86.229999 78.609999) (end 87.499999 79.879999) (width 1) (layer B.Cu) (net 27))
 (segment (start 87.499999 79.879999) (end 87.499999 80.682001) (width 1) (layer B.Cu) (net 27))
 (segment (start 87.499999 80.682001) (end 88.227999 81.410001) (width 1) (layer B.Cu) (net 27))
 (segment (start 123.87 77.47) (end 124.67 78.27) (width 1) (layer B.Cu) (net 28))
 (segment (start 115.57 77.47) (end 123.87 77.47) (width 1) (layer B.Cu) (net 28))
 (segment (start 91.44 91.44) (end 96.52 96.52) (width 1) (layer B.Cu) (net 30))
 (segment (start 93.98 99.06) (end 93.98 110.49) (width 1) (layer B.Cu) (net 30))
 (segment (start 96.52 96.52) (end 93.98 99.06) (width 1) (layer B.Cu) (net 30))
 (segment (start 123.770001 74.830001) (end 124.67 75.73) (width 1) (layer B.Cu) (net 30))
 (segment (start 130.81 74.93) (end 125.73 69.85) (width 1) (layer B.Cu) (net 30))
 (segment (start 125.73 69.85) (end 123.19 69.85) (width 1) (layer B.Cu) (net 30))
 (segment (start 130.81 110.353998) (end 130.81 74.93) (width 1) (layer B.Cu) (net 30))
 (segment (start 124.67 108.84) (end 123.397208 108.84) (width 1) (layer B.Cu) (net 30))
 (segment (start 123.397208 108.84) (end 123.069999 109.167209) (width 1) (layer B.Cu) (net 30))
 (segment (start 123.069999 69.970001) (end 121.799999 69.970001) (width 1) (layer B.Cu) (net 30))
 (segment (start 123.069999 109.167209) (end 123.069999 112.750001) (width 1) (layer B.Cu) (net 30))
 (segment (start 121.799999 72.859999) (end 123.770001 74.830001) (width 1) (layer B.Cu) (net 30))
 (segment (start 123.069999 112.750001) (end 124.551997 114.231999) (width 1) (layer B.Cu) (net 30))
 (segment (start 121.799999 69.970001) (end 121.799999 72.859999) (width 1) (layer B.Cu) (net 30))
 (segment (start 124.551997 114.231999) (end 126.931999 114.231999) (width 1) (layer B.Cu) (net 30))
 (segment (start 123.19 69.85) (end 123.069999 69.970001) (width 1) (layer B.Cu) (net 30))
 (segment (start 126.931999 114.231999) (end 130.81 110.353998) (width 1) (layer B.Cu) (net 30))
 (segment (start 63.569991 95.747061) (end 63.569991 74.860009) (width 1) (layer B.Cu) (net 30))
 (segment (start 85.182931 117.360001) (end 63.569991 95.747061) (width 1) (layer B.Cu) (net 30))
 (segment (start 115.797071 117.360001) (end 97.269999 117.360001) (width 1) (layer B.Cu) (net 30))
 (segment (start 123.397208 108.84) (end 123.397208 109.759864) (width 1) (layer B.Cu) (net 30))
 (segment (start 123.397208 109.759864) (end 115.797071 117.360001) (width 1) (layer B.Cu) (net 30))
 (segment (start 63.569991 74.860009) (end 67.31 71.12) (width 1) (layer B.Cu) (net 30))
 (segment (start 82.55 73.186443) (end 82.55 73.66) (width 1) (layer B.Cu) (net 30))
 (segment (start 80.483557 71.12) (end 82.55 73.186443) (width 1) (layer B.Cu) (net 30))
 (segment (start 67.31 71.12) (end 80.483557 71.12) (width 1) (layer B.Cu) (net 30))
 (segment (start 93.98 110.49) (end 97.79 110.49) (width 1) (layer B.Cu) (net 30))
 (segment (start 97.79 110.49) (end 97.79 110.49) (width 1) (layer B.Cu) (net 30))
 (via (at 97.79 110.49) (size 0.8) (drill 0.4) (layers F.Cu B.Cu) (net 30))
 (segment (start 97.269999 117.360001) (end 85.182931 117.360001) (width 1) (layer B.Cu) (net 30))
 (via (at 97.269999 117.360001) (size 0.8) (drill 0.4) (layers F.Cu B.Cu) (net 30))
 (segment (start 97.79 116.84) (end 97.269999 117.360001) (width 1) (layer F.Cu) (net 30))
 (segment (start 97.79 110.49) (end 97.79 116.84) (width 1) (layer F.Cu) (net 30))
 (segment (start 118.58 106.21) (end 124.67 106.21) (width 1) (layer B.Cu) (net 31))
 (segment (start 118.11 106.68) (end 118.58 106.21) (width 1) (layer B.Cu) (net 31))
 (segment (start 118.11 113.350002) (end 118.11 106.68) (width 1) (layer B.Cu) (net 31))
 (segment (start 91.48 115.49) (end 115.970002 115.49) (width 1) (layer B.Cu) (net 31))
 (segment (start 115.970002 115.49) (end 118.11 113.350002) (width 1) (layer B.Cu) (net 31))
 (segment (start 76.2 98.53) (end 76.2 100.33) (width 1) (layer B.Cu) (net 36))
 (segment (start 70.609999 92.939999) (end 76.2 98.53) (width 1) (layer B.Cu) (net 36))
 (segment (start 70.079999 92.939999) (end 70.609999 92.939999) (width 1) (layer B.Cu) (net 36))
 (segment (start 68.58 91.44) (end 70.079999 92.939999) (width 1) (layer B.Cu) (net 36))
 (segment (start 87.63 100.33) (end 88.9 101.6) (width 1) (layer B.Cu) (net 37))
 (segment (start 83.82 100.33) (end 87.63 100.33) (width 1) (layer B.Cu) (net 37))
 (segment (start 83.020001 99.530001) (end 83.82 100.33) (width 1) (layer B.Cu) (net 37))
 (segment (start 80.240001 96.750001) (end 83.020001 99.530001) (width 1) (layer B.Cu) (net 37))
 (segment (start 80.240001 87.860001) (end 80.240001 96.750001) (width 1) (layer B.Cu) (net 37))
 (segment (start 77.47 85.09) (end 80.240001 87.860001) (width 1) (layer B.Cu) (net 37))
 (segment (start 88.9 85.09) (end 87.790011 86.199989) (width 1) (layer B.Cu) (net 38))
 (segment (start 89.712799 98.247201) (end 88.9 99.06) (width 1) (layer B.Cu) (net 38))
 (segment (start 90.412801 97.547199) (end 89.712799 98.247201) (width 1) (layer B.Cu) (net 38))
 (segment (start 90.412801 95.492801) (end 90.412801 97.547199) (width 1) (layer B.Cu) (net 38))
 (segment (start 87.790011 92.870011) (end 90.412801 95.492801) (width 1) (layer B.Cu) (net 38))
 (segment (start 87.790011 86.199989) (end 87.790011 92.870011) (width 1) (layer B.Cu) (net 38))
 (segment (start 87.750528 99.06) (end 88.9 99.06) (width 1) (layer B.Cu) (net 38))
 (segment (start 82.389989 93.699461) (end 87.750528 99.06) (width 1) (layer B.Cu) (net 38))
 (segment (start 82.389989 88.312919) (end 82.389989 93.699461) (width 1) (layer B.Cu) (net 38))
 (segment (start 81.28 87.20293) (end 82.389989 88.312919) (width 1) (layer B.Cu) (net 38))
 (segment (start 81.28 85.09) (end 81.28 87.20293) (width 1) (layer B.Cu) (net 38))
 (segment (start 81.28 80.01) (end 85.09 80.01) (width 1) (layer B.Cu) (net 39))
 (segment (start 84.390001 80.709999) (end 85.09 80.01) (width 1) (layer B.Cu) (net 39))
 (segment (start 83.589999 81.510001) (end 84.390001 80.709999) (width 1) (layer B.Cu) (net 39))
 (segment (start 83.589999 92.800001) (end 83.589999 81.510001) (width 1) (layer B.Cu) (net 39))
 (segment (start 87.309998 96.52) (end 83.589999 92.800001) (width 1) (layer B.Cu) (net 39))
 (segment (start 88.9 96.52) (end 87.309998 96.52) (width 1) (layer B.Cu) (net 39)))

